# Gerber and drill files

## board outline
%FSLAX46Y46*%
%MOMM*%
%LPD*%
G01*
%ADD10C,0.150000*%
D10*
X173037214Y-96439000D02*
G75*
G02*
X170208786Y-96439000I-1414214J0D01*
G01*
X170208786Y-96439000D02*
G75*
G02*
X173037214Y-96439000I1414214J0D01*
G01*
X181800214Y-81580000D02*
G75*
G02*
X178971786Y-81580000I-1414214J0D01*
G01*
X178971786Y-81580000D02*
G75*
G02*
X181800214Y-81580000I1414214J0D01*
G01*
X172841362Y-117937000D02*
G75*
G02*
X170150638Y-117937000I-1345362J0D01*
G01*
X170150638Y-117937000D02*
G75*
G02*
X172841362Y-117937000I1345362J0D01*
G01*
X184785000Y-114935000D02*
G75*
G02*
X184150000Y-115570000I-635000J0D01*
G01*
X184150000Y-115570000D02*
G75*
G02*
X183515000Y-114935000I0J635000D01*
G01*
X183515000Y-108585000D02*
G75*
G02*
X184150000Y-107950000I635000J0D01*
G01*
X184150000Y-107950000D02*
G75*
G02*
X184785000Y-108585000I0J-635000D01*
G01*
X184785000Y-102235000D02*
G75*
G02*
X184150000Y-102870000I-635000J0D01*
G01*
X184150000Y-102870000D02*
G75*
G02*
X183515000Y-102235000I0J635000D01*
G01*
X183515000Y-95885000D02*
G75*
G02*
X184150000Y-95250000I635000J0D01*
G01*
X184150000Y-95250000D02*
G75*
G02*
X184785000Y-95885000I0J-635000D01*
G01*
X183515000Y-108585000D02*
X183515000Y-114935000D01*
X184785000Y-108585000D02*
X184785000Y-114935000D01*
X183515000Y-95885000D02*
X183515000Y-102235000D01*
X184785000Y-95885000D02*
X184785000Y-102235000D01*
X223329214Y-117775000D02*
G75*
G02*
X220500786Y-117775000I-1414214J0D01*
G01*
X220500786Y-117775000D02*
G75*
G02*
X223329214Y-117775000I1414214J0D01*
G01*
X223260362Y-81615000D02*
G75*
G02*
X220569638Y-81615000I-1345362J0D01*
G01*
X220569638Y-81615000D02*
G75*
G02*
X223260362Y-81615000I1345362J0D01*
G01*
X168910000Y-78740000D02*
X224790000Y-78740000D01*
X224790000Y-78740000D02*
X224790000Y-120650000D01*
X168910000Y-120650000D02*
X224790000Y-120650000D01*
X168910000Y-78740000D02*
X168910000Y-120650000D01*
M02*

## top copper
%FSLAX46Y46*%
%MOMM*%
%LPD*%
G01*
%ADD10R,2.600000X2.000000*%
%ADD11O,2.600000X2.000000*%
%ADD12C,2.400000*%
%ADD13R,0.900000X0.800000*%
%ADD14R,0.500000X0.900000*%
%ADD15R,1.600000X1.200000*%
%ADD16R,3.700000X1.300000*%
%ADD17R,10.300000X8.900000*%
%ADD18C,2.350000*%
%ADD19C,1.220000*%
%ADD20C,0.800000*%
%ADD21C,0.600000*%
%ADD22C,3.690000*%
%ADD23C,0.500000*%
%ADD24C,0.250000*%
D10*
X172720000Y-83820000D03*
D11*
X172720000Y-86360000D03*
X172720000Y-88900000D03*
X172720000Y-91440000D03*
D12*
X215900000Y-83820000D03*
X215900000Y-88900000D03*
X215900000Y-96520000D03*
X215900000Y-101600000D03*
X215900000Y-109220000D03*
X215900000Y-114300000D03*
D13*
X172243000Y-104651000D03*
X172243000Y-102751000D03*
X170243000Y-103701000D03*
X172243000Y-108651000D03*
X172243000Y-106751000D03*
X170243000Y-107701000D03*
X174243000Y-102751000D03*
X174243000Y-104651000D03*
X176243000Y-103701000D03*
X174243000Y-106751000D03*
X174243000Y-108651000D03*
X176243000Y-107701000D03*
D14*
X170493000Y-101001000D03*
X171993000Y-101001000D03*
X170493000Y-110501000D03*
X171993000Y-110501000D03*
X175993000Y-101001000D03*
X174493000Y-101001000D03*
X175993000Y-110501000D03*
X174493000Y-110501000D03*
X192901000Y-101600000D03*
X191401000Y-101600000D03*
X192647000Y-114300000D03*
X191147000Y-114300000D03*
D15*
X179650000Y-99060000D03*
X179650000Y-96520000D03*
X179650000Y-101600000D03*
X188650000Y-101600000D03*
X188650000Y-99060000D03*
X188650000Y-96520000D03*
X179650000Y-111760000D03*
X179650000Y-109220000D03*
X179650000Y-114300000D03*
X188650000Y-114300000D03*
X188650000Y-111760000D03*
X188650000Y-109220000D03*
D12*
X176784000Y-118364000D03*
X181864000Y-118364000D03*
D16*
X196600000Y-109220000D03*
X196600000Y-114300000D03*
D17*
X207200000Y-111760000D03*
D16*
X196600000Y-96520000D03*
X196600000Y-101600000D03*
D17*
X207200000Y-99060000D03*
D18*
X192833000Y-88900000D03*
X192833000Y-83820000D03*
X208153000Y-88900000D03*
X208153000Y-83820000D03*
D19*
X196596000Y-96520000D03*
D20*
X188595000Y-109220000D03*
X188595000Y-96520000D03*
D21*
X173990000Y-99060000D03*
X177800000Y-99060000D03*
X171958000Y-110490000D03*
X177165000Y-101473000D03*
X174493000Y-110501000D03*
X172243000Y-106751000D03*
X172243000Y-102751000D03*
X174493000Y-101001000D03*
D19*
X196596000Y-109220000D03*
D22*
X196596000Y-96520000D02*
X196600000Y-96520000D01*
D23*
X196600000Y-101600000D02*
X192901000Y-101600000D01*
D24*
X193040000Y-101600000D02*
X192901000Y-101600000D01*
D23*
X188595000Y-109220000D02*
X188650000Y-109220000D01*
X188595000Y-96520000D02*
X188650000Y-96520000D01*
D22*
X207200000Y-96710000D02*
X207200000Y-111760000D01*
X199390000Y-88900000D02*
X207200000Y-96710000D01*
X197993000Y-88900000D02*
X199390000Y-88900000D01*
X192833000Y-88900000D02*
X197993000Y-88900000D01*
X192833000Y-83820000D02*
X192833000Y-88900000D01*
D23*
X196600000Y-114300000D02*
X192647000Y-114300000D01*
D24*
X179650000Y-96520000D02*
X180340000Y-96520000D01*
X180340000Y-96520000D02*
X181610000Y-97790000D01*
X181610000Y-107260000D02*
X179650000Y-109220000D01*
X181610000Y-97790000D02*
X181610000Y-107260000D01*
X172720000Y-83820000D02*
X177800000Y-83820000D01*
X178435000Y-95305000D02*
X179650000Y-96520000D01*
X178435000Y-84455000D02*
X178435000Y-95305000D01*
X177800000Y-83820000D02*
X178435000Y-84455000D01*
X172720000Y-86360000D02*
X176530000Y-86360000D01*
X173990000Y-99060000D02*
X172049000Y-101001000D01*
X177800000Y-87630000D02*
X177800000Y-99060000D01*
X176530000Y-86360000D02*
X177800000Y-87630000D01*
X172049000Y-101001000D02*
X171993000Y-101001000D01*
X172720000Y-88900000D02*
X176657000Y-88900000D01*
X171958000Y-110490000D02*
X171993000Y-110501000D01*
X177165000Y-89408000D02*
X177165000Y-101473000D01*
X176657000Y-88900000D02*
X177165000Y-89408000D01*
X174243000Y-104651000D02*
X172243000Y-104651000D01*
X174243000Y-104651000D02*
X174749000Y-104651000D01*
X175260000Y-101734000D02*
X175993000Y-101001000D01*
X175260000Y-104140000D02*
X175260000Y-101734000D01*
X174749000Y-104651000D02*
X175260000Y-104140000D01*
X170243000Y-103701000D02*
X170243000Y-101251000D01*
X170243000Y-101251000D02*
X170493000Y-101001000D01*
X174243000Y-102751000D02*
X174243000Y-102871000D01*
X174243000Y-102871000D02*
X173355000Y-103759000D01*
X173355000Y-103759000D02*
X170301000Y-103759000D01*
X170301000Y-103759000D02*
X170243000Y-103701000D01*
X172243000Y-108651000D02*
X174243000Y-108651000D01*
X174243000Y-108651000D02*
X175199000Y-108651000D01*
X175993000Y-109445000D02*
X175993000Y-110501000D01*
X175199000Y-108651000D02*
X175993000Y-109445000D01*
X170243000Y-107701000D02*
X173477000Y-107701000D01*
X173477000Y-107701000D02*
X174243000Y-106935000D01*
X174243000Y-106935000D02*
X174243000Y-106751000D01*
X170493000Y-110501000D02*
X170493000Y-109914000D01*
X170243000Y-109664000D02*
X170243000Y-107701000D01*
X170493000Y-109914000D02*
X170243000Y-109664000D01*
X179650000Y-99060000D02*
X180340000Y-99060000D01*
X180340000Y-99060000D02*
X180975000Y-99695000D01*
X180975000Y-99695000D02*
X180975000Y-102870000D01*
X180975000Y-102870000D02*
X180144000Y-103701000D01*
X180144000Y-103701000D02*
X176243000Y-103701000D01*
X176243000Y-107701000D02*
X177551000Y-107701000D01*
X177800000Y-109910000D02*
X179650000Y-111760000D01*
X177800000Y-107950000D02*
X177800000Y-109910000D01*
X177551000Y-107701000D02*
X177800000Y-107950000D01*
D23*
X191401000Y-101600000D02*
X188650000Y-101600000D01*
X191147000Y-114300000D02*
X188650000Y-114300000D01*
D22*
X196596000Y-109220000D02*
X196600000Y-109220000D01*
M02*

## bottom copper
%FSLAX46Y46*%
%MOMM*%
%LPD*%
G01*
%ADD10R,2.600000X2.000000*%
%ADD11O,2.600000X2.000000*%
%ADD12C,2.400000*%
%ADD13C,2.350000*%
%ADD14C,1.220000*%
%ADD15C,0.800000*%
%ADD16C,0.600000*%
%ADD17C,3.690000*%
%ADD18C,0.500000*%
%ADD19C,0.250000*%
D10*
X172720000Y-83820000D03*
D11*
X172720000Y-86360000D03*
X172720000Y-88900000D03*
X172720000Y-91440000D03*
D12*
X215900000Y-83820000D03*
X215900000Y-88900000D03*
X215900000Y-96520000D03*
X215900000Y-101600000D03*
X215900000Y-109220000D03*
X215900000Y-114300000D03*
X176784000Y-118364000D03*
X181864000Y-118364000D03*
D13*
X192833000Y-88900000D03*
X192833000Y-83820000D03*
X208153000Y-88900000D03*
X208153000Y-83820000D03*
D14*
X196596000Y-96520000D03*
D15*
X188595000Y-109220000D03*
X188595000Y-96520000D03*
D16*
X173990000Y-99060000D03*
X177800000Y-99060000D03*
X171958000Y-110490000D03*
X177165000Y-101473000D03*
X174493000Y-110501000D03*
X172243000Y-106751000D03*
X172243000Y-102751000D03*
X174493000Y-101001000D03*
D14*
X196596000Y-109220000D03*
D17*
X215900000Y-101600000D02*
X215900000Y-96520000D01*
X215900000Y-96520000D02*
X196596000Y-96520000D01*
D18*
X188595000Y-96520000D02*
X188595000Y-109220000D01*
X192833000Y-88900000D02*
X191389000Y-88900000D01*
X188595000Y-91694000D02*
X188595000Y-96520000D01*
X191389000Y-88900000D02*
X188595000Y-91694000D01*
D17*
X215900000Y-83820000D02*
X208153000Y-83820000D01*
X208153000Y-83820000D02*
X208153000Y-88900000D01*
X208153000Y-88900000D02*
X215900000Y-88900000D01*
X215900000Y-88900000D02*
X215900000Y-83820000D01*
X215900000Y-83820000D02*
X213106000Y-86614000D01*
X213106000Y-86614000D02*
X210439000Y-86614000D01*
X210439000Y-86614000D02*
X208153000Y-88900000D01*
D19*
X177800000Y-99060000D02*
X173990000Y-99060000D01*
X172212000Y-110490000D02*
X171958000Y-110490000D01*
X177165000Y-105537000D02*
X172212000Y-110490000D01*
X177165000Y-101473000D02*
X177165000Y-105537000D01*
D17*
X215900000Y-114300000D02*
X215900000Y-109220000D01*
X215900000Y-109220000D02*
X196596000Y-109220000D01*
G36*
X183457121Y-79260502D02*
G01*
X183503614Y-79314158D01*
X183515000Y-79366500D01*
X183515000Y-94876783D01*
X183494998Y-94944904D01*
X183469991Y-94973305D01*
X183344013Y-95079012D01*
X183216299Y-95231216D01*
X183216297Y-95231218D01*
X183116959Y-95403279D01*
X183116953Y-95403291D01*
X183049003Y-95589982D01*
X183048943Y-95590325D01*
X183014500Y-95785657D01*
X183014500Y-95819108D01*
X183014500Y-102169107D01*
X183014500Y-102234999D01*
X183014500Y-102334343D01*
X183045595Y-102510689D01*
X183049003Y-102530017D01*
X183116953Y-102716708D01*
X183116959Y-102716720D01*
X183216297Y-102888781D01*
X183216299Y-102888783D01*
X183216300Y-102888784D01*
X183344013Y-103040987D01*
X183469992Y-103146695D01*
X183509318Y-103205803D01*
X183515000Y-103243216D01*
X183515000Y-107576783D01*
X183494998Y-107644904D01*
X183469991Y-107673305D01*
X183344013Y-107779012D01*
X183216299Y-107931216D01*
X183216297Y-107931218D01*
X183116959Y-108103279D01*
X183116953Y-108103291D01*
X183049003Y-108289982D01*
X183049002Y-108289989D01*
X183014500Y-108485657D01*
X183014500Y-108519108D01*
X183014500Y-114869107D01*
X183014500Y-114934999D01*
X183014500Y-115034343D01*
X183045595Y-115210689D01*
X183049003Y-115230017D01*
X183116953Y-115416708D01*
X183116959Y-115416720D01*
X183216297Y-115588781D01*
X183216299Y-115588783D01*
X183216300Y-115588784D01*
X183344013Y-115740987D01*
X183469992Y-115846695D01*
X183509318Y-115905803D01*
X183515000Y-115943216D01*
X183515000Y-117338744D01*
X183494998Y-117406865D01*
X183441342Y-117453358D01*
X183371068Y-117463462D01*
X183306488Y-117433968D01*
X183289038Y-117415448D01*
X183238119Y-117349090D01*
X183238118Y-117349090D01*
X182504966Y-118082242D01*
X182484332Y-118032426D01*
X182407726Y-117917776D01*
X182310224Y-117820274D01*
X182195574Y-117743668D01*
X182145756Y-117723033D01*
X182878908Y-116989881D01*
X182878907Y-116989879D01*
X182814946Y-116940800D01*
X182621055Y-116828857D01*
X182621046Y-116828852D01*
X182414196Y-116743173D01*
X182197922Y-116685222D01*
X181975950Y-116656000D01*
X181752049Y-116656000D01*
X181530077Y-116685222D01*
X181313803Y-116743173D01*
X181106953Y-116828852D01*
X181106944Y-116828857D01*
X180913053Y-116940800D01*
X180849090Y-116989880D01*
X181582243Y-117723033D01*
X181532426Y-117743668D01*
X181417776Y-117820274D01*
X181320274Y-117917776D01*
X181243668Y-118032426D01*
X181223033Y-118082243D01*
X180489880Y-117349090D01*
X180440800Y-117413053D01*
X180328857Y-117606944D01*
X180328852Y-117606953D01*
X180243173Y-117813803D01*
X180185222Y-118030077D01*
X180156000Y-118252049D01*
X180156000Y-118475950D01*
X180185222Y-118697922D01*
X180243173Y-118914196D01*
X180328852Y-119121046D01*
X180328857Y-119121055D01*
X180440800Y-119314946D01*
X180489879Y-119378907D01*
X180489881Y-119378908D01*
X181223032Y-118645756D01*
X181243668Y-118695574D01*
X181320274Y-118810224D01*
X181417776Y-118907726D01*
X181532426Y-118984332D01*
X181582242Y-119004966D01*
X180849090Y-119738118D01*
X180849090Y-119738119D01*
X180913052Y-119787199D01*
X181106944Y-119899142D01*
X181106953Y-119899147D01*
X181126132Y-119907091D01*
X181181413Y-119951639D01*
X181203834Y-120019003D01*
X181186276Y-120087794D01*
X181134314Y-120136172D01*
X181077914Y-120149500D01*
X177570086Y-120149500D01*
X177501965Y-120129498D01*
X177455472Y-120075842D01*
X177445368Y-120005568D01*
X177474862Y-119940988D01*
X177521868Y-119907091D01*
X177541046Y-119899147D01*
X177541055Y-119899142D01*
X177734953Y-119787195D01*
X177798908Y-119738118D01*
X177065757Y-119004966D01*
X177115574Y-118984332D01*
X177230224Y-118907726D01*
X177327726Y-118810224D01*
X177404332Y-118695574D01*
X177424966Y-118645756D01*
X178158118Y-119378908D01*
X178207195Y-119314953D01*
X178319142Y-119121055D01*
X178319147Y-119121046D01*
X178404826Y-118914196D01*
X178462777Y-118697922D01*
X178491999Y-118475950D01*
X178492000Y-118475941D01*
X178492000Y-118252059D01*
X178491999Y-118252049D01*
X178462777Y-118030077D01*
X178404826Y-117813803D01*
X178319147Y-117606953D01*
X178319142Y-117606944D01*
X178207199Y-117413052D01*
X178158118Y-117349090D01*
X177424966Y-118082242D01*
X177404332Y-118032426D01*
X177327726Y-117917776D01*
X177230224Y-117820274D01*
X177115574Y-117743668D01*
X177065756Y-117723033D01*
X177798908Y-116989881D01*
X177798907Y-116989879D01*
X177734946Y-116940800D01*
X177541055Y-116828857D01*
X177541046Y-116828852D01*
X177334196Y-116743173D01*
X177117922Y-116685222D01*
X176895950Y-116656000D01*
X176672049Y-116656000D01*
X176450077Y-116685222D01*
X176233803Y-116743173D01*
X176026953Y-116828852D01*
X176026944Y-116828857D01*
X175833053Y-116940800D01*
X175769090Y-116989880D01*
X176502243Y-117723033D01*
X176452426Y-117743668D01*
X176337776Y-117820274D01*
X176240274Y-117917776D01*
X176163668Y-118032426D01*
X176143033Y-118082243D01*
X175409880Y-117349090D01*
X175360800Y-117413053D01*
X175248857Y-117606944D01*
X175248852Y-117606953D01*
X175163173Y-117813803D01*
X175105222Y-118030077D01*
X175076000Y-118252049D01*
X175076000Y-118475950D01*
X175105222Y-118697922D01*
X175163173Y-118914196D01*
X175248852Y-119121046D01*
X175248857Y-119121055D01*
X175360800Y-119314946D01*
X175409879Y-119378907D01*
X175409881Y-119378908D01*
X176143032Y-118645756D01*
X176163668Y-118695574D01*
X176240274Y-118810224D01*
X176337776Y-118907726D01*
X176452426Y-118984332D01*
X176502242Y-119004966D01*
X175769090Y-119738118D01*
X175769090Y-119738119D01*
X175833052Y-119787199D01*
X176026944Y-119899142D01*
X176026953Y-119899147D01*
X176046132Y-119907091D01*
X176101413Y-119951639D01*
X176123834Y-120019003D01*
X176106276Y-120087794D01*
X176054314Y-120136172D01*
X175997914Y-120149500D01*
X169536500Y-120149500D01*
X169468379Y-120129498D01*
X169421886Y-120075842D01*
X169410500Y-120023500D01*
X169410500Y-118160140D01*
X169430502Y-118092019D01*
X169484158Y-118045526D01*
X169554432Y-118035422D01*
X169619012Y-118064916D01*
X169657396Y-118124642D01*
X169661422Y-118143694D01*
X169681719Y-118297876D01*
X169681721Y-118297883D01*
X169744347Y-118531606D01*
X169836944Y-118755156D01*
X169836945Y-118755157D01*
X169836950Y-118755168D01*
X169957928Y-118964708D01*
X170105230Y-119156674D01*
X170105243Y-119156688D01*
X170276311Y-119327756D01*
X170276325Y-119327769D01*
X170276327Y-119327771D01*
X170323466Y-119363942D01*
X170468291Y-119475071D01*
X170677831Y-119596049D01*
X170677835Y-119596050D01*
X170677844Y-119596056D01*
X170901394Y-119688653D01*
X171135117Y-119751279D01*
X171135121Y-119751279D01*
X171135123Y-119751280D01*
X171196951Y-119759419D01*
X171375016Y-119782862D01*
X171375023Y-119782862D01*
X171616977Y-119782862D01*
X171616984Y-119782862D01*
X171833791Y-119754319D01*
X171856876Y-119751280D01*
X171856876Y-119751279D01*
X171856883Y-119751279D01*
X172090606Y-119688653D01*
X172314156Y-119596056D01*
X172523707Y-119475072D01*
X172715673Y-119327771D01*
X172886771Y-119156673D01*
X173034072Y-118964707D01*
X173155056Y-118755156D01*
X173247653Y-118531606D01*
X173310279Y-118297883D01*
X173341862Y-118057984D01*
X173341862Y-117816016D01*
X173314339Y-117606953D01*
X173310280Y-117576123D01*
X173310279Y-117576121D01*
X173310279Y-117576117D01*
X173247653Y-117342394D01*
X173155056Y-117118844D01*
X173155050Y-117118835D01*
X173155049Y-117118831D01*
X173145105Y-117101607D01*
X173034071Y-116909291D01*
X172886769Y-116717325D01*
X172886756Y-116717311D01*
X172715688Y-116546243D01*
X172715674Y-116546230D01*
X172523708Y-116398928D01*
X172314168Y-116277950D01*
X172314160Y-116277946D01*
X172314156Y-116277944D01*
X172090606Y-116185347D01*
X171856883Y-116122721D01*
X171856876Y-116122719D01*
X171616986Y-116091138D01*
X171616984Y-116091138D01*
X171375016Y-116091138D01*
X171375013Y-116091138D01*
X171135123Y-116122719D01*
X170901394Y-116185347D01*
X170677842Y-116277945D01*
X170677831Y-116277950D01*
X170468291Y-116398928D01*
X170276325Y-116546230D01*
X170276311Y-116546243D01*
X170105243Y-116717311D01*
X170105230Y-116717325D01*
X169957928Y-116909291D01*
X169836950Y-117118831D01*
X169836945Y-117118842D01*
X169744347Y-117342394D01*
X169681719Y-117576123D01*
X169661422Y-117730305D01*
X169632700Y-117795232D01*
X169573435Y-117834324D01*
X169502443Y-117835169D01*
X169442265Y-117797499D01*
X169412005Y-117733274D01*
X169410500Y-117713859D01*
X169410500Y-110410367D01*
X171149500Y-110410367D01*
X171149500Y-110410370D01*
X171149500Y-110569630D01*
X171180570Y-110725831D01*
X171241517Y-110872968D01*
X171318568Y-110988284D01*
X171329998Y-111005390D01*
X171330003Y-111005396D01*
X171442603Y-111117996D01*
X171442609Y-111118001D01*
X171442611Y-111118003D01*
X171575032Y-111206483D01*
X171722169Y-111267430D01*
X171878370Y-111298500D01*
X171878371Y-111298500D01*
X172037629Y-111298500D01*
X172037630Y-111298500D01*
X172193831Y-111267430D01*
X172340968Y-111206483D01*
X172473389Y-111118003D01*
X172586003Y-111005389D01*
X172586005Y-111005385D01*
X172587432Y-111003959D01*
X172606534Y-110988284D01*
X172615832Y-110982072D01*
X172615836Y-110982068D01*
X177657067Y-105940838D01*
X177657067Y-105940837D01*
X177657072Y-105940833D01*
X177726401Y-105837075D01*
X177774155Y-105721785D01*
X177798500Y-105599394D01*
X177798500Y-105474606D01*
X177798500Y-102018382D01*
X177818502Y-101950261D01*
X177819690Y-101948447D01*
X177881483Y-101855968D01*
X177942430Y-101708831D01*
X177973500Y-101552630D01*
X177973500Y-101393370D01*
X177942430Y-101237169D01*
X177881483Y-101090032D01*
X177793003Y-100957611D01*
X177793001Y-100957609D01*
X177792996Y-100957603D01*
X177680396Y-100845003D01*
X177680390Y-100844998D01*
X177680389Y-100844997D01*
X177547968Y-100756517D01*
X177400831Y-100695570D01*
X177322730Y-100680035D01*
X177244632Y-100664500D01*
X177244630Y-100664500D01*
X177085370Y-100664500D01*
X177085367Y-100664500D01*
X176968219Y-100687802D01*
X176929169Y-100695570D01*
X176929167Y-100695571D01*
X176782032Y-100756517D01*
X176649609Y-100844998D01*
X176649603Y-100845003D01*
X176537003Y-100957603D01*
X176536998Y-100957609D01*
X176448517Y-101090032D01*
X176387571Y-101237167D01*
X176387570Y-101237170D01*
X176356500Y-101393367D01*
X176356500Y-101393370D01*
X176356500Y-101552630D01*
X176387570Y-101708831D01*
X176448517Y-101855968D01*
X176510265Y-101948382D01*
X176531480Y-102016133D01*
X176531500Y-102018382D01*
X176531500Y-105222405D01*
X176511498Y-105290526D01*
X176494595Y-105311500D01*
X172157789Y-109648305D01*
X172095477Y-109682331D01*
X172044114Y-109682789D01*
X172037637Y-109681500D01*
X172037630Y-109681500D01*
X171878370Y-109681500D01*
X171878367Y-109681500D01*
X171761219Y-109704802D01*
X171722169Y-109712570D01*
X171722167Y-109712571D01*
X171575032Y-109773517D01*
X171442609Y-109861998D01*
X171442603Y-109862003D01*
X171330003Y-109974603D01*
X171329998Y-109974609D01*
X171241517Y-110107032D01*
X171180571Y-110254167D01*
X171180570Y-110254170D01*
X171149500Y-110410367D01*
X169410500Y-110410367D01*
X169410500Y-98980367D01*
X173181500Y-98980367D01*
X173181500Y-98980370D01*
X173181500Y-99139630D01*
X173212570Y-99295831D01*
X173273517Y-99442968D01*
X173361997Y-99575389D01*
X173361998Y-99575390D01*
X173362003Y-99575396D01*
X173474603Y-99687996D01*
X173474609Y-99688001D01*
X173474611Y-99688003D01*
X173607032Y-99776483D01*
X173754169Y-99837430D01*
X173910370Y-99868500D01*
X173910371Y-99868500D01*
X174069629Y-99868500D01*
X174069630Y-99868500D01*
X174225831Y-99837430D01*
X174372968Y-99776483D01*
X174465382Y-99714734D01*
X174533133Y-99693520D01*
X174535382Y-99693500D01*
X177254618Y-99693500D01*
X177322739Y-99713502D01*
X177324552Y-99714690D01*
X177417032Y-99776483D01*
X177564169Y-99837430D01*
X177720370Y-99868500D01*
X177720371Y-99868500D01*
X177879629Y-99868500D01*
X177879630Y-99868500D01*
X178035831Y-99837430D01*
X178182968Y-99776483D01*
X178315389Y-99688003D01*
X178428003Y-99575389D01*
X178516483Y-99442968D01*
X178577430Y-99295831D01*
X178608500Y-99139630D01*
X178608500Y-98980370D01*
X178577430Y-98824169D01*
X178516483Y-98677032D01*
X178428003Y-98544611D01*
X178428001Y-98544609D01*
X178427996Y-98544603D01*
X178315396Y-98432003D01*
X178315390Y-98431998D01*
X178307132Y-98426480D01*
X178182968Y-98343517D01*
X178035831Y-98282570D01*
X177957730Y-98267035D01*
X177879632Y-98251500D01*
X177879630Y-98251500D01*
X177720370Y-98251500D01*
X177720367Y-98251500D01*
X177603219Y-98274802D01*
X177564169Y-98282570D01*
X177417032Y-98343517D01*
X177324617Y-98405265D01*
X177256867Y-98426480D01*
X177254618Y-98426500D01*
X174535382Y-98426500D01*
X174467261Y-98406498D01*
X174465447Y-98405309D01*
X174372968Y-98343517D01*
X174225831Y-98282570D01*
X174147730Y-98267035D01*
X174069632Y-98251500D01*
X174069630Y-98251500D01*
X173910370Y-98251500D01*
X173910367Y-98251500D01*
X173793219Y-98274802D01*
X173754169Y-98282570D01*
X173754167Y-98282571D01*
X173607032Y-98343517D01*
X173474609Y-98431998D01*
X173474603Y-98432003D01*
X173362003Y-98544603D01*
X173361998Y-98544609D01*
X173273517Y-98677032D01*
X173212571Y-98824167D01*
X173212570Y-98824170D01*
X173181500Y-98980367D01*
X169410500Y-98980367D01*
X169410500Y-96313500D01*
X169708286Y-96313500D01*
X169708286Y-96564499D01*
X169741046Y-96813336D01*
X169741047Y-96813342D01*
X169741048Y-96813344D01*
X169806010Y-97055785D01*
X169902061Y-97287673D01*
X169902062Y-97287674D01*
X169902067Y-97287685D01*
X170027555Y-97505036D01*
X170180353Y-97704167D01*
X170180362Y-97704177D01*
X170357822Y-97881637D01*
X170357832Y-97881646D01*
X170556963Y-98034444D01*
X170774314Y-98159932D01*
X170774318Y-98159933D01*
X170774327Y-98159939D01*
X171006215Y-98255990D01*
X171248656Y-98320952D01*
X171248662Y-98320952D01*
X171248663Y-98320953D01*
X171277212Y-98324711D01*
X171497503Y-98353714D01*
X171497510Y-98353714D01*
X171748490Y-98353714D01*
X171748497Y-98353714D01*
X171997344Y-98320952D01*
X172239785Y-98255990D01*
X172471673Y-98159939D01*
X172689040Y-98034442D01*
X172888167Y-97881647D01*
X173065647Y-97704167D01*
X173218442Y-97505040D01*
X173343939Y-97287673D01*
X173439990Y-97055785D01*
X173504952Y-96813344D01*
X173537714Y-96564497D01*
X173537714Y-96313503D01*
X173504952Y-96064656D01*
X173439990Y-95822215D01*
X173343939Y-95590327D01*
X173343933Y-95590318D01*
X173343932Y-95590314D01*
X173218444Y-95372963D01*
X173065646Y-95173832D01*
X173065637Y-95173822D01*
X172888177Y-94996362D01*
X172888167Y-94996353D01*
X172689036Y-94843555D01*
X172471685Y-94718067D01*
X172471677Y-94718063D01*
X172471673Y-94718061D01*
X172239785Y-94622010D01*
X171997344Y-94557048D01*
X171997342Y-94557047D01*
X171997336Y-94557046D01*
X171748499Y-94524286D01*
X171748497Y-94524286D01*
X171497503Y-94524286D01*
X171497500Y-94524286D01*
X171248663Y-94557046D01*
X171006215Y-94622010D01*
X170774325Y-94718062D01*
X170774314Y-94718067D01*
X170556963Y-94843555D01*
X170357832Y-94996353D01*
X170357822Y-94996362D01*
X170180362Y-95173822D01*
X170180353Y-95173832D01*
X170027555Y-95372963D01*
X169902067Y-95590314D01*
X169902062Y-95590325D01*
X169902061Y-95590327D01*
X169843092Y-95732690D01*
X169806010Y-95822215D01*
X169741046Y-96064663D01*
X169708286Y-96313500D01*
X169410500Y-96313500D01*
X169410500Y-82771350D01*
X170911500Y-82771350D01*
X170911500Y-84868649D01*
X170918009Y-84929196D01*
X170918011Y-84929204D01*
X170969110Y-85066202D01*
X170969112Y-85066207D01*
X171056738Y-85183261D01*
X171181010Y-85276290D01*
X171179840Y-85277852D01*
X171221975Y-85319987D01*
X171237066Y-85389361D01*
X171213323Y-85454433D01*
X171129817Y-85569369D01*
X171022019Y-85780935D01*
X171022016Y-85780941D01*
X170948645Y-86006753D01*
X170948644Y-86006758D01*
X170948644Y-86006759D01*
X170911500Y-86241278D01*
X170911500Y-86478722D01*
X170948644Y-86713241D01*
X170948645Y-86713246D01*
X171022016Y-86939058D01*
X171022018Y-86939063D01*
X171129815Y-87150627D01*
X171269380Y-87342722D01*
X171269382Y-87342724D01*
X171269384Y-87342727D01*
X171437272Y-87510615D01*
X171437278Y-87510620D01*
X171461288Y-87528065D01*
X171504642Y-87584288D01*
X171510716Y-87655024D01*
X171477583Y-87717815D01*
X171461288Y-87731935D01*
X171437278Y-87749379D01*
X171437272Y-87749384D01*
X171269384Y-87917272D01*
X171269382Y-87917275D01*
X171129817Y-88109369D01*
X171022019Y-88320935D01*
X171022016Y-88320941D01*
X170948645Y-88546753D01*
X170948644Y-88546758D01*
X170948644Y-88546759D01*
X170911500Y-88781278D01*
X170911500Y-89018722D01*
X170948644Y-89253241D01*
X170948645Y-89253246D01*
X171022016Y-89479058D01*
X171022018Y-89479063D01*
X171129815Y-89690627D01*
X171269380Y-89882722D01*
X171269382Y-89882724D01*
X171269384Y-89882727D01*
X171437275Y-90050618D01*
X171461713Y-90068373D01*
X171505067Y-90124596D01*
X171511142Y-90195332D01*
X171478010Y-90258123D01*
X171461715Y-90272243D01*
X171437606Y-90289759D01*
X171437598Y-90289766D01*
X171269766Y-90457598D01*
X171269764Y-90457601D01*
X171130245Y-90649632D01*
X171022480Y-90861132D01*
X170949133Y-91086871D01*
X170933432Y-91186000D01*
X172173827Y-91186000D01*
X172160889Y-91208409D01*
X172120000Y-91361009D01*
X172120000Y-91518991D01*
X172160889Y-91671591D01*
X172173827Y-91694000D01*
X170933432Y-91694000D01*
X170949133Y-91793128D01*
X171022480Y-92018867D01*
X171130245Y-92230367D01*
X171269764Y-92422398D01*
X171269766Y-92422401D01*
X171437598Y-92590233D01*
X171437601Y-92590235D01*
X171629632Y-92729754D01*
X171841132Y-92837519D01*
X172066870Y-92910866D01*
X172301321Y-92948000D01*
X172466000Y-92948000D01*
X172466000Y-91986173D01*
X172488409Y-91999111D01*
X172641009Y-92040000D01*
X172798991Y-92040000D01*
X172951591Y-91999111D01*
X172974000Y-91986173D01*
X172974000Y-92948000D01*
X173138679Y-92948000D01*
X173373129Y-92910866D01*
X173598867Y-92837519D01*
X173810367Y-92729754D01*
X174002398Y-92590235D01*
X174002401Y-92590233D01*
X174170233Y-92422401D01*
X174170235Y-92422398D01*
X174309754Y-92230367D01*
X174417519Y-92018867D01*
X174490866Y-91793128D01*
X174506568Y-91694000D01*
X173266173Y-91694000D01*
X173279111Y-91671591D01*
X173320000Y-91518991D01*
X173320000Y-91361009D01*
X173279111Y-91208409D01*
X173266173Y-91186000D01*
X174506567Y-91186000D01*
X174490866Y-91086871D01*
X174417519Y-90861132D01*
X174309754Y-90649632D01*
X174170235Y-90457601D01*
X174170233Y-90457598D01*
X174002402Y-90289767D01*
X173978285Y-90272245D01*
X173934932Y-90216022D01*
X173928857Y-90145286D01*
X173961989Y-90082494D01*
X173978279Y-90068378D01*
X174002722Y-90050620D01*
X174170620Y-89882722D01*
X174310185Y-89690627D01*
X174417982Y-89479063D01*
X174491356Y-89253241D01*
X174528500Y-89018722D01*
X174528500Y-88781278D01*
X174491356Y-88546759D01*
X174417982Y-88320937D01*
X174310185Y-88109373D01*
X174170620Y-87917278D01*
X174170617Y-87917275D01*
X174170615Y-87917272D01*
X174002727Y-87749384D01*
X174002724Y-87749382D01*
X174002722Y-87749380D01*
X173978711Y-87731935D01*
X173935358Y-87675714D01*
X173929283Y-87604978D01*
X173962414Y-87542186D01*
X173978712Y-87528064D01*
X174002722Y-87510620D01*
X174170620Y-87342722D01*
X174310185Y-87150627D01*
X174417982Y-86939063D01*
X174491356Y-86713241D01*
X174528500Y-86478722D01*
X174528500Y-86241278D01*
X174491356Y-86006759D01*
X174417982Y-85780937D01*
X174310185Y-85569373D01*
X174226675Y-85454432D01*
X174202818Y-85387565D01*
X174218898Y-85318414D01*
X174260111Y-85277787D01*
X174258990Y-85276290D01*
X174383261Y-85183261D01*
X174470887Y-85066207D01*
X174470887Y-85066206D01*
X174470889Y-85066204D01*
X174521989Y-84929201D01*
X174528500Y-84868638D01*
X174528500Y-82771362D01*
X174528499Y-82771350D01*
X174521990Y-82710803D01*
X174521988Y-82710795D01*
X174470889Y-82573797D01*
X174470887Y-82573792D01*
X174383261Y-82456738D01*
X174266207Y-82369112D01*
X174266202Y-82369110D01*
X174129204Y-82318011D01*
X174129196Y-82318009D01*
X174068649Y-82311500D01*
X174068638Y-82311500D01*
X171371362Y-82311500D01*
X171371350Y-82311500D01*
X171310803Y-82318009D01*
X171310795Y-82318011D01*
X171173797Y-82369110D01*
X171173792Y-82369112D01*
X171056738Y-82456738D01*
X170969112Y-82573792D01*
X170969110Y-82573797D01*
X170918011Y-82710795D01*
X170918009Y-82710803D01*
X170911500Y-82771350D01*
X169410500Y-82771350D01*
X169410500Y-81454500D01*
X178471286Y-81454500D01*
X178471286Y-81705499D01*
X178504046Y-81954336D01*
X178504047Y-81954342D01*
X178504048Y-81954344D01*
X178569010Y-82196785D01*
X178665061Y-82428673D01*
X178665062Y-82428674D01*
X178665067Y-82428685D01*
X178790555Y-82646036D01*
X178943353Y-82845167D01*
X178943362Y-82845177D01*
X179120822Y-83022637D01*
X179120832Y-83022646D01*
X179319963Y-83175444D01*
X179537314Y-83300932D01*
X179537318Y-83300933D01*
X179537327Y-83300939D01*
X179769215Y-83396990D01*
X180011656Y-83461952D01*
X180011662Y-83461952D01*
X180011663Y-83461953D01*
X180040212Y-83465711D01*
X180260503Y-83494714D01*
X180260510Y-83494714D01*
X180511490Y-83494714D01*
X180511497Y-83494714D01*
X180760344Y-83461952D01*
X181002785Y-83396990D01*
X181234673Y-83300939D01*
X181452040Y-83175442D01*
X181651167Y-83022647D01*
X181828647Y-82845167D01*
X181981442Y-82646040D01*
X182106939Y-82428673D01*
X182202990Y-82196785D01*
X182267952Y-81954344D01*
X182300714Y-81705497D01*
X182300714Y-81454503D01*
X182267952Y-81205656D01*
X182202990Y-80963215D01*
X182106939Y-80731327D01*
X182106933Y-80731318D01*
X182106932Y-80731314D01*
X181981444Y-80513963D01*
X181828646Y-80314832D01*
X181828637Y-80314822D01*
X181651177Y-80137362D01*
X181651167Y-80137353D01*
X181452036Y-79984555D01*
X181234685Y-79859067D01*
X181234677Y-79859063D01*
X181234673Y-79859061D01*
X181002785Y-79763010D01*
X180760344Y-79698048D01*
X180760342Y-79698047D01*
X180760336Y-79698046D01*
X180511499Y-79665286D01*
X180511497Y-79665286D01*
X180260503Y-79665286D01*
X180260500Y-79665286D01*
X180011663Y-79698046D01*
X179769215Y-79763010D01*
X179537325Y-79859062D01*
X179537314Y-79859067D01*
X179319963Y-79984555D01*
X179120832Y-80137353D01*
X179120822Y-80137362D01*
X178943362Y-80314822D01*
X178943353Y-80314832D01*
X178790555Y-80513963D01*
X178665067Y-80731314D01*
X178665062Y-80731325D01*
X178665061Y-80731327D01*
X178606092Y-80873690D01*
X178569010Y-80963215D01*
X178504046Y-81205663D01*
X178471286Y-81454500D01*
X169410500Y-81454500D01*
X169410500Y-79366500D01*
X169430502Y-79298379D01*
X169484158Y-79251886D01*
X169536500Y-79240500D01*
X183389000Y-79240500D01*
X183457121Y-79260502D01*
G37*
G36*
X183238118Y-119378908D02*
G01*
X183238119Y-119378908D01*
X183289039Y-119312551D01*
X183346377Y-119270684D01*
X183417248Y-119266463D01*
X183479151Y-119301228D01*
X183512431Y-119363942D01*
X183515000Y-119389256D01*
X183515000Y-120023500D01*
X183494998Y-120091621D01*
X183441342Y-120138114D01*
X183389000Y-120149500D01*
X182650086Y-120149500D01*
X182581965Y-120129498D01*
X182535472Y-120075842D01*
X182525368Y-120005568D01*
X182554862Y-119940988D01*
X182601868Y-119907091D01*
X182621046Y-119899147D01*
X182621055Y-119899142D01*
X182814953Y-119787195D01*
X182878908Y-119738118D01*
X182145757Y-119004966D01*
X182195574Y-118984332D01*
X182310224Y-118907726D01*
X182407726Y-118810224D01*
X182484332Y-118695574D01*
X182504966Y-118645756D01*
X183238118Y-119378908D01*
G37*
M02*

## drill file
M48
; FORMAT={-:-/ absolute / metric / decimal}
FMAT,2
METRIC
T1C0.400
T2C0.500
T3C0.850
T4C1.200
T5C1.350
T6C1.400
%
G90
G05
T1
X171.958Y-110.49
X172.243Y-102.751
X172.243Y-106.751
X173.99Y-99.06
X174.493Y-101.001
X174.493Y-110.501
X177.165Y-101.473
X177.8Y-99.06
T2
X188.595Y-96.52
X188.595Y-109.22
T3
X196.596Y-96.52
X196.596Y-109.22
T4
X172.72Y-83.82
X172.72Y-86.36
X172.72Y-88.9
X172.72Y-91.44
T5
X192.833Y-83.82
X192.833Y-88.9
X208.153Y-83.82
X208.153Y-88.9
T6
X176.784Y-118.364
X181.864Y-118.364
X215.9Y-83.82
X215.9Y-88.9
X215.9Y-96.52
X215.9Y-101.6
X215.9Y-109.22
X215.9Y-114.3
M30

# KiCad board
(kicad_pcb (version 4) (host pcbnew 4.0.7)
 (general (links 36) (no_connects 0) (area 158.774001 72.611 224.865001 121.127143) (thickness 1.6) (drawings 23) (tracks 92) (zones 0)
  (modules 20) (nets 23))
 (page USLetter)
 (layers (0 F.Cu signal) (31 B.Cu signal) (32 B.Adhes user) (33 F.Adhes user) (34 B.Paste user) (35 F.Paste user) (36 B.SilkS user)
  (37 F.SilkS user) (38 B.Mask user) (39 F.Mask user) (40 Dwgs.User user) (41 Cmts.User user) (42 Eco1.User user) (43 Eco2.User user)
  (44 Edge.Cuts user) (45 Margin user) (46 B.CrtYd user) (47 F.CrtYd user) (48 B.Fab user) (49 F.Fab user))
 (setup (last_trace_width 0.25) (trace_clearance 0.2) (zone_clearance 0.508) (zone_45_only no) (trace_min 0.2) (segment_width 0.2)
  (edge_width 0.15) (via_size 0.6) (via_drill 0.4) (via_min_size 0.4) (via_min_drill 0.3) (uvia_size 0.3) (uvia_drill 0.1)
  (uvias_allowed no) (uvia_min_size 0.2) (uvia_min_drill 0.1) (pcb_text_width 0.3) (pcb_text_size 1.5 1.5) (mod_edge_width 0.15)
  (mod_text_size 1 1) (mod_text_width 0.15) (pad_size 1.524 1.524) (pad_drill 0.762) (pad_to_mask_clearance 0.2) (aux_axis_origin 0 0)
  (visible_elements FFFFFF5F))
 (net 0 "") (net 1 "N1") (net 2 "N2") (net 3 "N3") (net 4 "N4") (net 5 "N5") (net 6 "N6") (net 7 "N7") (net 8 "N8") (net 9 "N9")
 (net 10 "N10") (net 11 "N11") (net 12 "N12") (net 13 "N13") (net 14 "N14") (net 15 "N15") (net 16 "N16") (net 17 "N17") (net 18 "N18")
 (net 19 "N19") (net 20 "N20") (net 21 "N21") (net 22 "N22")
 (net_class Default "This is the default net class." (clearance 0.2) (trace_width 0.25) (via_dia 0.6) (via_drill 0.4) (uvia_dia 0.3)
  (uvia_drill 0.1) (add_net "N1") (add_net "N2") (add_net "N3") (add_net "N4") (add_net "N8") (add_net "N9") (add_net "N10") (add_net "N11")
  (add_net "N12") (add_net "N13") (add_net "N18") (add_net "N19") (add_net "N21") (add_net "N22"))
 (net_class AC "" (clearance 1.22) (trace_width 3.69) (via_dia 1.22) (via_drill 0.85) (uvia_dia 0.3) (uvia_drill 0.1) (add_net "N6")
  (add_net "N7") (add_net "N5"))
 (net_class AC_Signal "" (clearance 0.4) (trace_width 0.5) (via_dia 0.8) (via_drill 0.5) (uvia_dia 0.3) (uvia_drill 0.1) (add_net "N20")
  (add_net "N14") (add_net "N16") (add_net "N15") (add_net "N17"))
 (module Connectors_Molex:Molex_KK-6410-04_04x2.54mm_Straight (layer F.Cu) (at 172.72 83.82 270)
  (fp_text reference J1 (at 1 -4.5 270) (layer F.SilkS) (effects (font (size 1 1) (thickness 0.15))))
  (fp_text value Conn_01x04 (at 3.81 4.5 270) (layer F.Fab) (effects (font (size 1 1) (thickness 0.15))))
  (pad 1 thru_hole rect (at 0 0 270) (size 2 2.6) (drill 1.2) (layers *.Cu *.Mask) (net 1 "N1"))
  (pad 2 thru_hole oval (at 2.54 0 270) (size 2 2.6) (drill 1.2) (layers *.Cu *.Mask) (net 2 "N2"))
  (pad 3 thru_hole oval (at 5.08 0 270) (size 2 2.6) (drill 1.2) (layers *.Cu *.Mask) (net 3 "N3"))
  (pad 4 thru_hole oval (at 7.62 0 270) (size 2 2.6) (drill 1.2) (layers *.Cu *.Mask) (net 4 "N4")))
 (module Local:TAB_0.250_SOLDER (layer F.Cu) (at 215.9 88.9 90)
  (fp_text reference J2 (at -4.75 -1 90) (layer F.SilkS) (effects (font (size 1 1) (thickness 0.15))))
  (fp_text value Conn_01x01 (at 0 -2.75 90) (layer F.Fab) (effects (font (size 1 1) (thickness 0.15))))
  (pad 1 thru_hole circle (at 5.08 0 90) (size 2.4 2.4) (drill 1.4) (layers *.Cu *.Mask) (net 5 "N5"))
  (pad 1 thru_hole circle (at 0 0 90) (size 2.4 2.4) (drill 1.4) (layers *.Cu *.Mask) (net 5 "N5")))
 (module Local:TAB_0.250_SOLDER (layer F.Cu) (at 215.9 101.6 90)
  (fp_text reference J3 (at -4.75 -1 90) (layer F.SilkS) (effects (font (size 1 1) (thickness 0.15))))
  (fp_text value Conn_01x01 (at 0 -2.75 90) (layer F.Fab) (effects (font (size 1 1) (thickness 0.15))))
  (pad 1 thru_hole circle (at 5.08 0 90) (size 2.4 2.4) (drill 1.4) (layers *.Cu *.Mask) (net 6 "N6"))
  (pad 1 thru_hole circle (at 0 0 90) (size 2.4 2.4) (drill 1.4) (layers *.Cu *.Mask) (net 6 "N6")))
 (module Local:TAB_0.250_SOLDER (layer F.Cu) (at 215.9 114.3 90)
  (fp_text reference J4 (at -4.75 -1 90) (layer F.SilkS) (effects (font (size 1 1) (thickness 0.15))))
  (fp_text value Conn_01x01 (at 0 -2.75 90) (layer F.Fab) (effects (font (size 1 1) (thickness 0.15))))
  (pad 1 thru_hole circle (at 5.08 0 90) (size 2.4 2.4) (drill 1.4) (layers *.Cu *.Mask) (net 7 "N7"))
  (pad 1 thru_hole circle (at 0 0 90) (size 2.4 2.4) (drill 1.4) (layers *.Cu *.Mask) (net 7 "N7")))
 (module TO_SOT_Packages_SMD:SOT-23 (layer F.Cu) (at 171.243 103.701 180)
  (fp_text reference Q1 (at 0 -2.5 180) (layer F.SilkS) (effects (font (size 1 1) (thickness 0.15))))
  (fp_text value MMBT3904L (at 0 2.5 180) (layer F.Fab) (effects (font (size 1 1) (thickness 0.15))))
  (pad 1 smd rect (at -1 -0.95 180) (size 0.9 0.8) (layers F.Cu F.Paste F.Mask) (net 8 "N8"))
  (pad 2 smd rect (at -1 0.95 180) (size 0.9 0.8) (layers F.Cu F.Paste F.Mask) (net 4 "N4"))
  (pad 3 smd rect (at 1 0 180) (size 0.9 0.8) (layers F.Cu F.Paste F.Mask) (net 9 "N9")))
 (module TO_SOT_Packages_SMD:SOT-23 (layer F.Cu) (at 171.243 107.701 180)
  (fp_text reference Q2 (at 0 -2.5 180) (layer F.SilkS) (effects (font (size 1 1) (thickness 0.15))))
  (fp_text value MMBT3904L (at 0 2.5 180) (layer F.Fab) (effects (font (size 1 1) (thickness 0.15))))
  (pad 1 smd rect (at -1 -0.95 180) (size 0.9 0.8) (layers F.Cu F.Paste F.Mask) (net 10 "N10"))
  (pad 2 smd rect (at -1 0.95 180) (size 0.9 0.8) (layers F.Cu F.Paste F.Mask) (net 4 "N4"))
  (pad 3 smd rect (at 1 0 180) (size 0.9 0.8) (layers F.Cu F.Paste F.Mask) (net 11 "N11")))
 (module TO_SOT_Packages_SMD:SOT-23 (layer F.Cu) (at 175.243 103.701)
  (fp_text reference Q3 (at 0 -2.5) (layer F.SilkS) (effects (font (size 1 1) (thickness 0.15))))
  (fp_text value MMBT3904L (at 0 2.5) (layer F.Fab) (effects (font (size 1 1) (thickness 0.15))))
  (pad 1 smd rect (at -1 -0.95) (size 0.9 0.8) (layers F.Cu F.Paste F.Mask) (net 9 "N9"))
  (pad 2 smd rect (at -1 0.95) (size 0.9 0.8) (layers F.Cu F.Paste F.Mask) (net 8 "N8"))
  (pad 3 smd rect (at 1 0) (size 0.9 0.8) (layers F.Cu F.Paste F.Mask) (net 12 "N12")))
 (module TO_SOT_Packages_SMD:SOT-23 (layer F.Cu) (at 175.243 107.701)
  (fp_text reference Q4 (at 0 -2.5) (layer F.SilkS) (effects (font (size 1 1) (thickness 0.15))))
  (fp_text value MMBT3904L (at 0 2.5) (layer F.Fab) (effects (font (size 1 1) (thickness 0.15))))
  (pad 1 smd rect (at -1 -0.95) (size 0.9 0.8) (layers F.Cu F.Paste F.Mask) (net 11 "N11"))
  (pad 2 smd rect (at -1 0.95) (size 0.9 0.8) (layers F.Cu F.Paste F.Mask) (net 10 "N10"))
  (pad 3 smd rect (at 1 0) (size 0.9 0.8) (layers F.Cu F.Paste F.Mask) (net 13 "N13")))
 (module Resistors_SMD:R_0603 (layer F.Cu) (at 171.243 101.001)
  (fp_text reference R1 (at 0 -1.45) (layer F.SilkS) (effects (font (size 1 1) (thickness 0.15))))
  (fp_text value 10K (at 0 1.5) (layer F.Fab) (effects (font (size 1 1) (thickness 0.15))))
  (pad 1 smd rect (at -0.75 0) (size 0.5 0.9) (layers F.Cu F.Paste F.Mask) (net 9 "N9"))
  (pad 2 smd rect (at 0.75 0) (size 0.5 0.9) (layers F.Cu F.Paste F.Mask) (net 2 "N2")))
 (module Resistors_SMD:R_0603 (layer F.Cu) (at 171.243 110.501)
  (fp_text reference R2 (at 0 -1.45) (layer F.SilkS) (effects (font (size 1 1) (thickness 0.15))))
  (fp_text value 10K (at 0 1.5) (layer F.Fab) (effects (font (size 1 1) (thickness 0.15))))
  (pad 1 smd rect (at -0.75 0) (size 0.5 0.9) (layers F.Cu F.Paste F.Mask) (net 11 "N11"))
  (pad 2 smd rect (at 0.75 0) (size 0.5 0.9) (layers F.Cu F.Paste F.Mask) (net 3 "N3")))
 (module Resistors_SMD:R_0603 (layer F.Cu) (at 175.243 101.001 180)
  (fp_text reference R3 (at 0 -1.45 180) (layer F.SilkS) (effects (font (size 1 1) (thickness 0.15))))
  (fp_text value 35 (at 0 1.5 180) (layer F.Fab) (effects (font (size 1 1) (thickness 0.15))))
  (pad 1 smd rect (at -0.75 0 180) (size 0.5 0.9) (layers F.Cu F.Paste F.Mask) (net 8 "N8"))
  (pad 2 smd rect (at 0.75 0 180) (size 0.5 0.9) (layers F.Cu F.Paste F.Mask) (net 4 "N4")))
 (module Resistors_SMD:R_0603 (layer F.Cu) (at 175.243 110.501 180)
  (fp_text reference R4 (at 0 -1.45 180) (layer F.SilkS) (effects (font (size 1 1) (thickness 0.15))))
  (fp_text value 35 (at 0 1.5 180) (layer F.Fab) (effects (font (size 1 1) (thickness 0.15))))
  (pad 1 smd rect (at -0.75 0 180) (size 0.5 0.9) (layers F.Cu F.Paste F.Mask) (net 10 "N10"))
  (pad 2 smd rect (at 0.75 0 180) (size 0.5 0.9) (layers F.Cu F.Paste F.Mask) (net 4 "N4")))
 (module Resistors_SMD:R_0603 (layer F.Cu) (at 192.151 101.6 180)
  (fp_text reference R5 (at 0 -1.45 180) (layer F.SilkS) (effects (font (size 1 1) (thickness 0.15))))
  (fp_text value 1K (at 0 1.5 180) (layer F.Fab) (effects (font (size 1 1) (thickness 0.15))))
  (pad 1 smd rect (at -0.75 0 180) (size 0.5 0.9) (layers F.Cu F.Paste F.Mask) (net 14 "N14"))
  (pad 2 smd rect (at 0.75 0 180) (size 0.5 0.9) (layers F.Cu F.Paste F.Mask) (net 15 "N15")))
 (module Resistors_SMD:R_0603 (layer F.Cu) (at 191.897 114.3 180)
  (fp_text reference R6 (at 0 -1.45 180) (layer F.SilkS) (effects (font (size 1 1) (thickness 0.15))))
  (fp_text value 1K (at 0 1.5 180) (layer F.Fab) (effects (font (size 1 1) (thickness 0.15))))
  (pad 1 smd rect (at -0.75 0 180) (size 0.5 0.9) (layers F.Cu F.Paste F.Mask) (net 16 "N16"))
  (pad 2 smd rect (at 0.75 0 180) (size 0.5 0.9) (layers F.Cu F.Paste F.Mask) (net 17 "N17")))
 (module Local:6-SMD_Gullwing (layer F.Cu) (at 184.15 99.06 270)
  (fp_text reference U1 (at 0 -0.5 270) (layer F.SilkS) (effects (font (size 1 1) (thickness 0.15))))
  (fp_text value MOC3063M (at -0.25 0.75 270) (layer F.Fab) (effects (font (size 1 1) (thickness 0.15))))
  (pad 2 smd rect (at 0 4.5 270) (size 1.2 1.6) (layers F.Cu F.Paste F.Mask) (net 12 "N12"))
  (pad 1 smd rect (at -2.54 4.5 270) (size 1.2 1.6) (layers F.Cu F.Paste F.Mask) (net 1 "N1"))
  (pad 3 smd rect (at 2.54 4.5 270) (size 1.2 1.6) (layers F.Cu F.Paste F.Mask) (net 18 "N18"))
  (pad 4 smd rect (at 2.54 -4.5 270) (size 1.2 1.6) (layers F.Cu F.Paste F.Mask) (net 15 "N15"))
  (pad 5 smd rect (at 0 -4.5 270) (size 1.2 1.6) (layers F.Cu F.Paste F.Mask) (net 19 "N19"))
  (pad 6 smd rect (at -2.54 -4.5 270) (size 1.2 1.6) (layers F.Cu F.Paste F.Mask) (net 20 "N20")))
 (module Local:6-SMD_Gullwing (layer F.Cu) (at 184.15 111.76 270)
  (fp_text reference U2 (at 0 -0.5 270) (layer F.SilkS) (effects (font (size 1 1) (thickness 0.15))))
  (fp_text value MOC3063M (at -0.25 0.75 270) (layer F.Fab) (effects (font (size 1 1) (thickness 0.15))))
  (pad 2 smd rect (at 0 4.5 270) (size 1.2 1.6) (layers F.Cu F.Paste F.Mask) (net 13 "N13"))
  (pad 1 smd rect (at -2.54 4.5 270) (size 1.2 1.6) (layers F.Cu F.Paste F.Mask) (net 1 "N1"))
  (pad 3 smd rect (at 2.54 4.5 270) (size 1.2 1.6) (layers F.Cu F.Paste F.Mask) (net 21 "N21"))
  (pad 4 smd rect (at 2.54 -4.5 270) (size 1.2 1.6) (layers F.Cu F.Paste F.Mask) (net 17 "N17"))
  (pad 5 smd rect (at 0 -4.5 270) (size 1.2 1.6) (layers F.Cu F.Paste F.Mask) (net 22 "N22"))
  (pad 6 smd rect (at -2.54 -4.5 270) (size 1.2 1.6) (layers F.Cu F.Paste F.Mask) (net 20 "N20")))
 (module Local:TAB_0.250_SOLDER (layer F.Cu) (at 181.864 118.364 180)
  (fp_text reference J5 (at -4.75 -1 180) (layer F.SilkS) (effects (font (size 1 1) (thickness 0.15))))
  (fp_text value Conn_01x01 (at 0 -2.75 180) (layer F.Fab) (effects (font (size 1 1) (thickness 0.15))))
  (pad 1 thru_hole circle (at 5.08 0 180) (size 2.4 2.4) (drill 1.4) (layers *.Cu *.Mask) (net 4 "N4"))
  (pad 1 thru_hole circle (at 0 0 180) (size 2.4 2.4) (drill 1.4) (layers *.Cu *.Mask) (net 4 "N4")))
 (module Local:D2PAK (layer F.Cu) (at 203.2 111.76 180)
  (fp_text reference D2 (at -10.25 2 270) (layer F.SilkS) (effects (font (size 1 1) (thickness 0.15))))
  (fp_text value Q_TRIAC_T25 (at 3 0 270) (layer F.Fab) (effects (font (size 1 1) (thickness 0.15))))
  (pad 1 smd rect (at 6.6 2.54 180) (size 3.7 1.3) (layers F.Cu F.Paste F.Mask) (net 7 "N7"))
  (pad 3 smd rect (at 6.6 -2.54 180) (size 3.7 1.3) (layers F.Cu F.Paste F.Mask) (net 16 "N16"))
  (pad 2 smd rect (at -4 0 180) (size 10.3 8.9) (layers F.Cu F.Paste F.Mask) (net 20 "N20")))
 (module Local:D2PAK (layer F.Cu) (at 203.2 99.06 180)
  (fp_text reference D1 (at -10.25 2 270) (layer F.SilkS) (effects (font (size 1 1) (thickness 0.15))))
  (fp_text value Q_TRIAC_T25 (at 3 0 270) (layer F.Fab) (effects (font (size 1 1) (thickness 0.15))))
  (pad 1 smd rect (at 6.6 2.54 180) (size 3.7 1.3) (layers F.Cu F.Paste F.Mask) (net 6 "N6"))
  (pad 3 smd rect (at 6.6 -2.54 180) (size 3.7 1.3) (layers F.Cu F.Paste F.Mask) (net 14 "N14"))
  (pad 2 smd rect (at -4 0 180) (size 10.3 8.9) (layers F.Cu F.Paste F.Mask) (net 20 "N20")))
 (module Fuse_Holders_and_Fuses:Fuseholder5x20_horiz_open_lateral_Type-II (layer F.Cu) (at 208.153 88.9 180)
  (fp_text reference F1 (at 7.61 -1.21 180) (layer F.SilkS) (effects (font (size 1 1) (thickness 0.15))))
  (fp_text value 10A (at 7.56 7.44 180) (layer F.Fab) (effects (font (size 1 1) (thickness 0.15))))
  (pad 2 thru_hole circle (at 15.32 0 180) (size 2.35 2.35) (drill 1.35) (layers *.Cu *.Mask) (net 20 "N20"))
  (pad 2 thru_hole circle (at 15.32 5.08 180) (size 2.35 2.35) (drill 1.35) (layers *.Cu *.Mask) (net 20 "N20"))
  (pad 1 thru_hole circle (at 0 0 180) (size 2.35 2.35) (drill 1.35) (layers *.Cu *.Mask) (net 5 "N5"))
  (pad 1 thru_hole circle (at 0 5.08 180) (size 2.35 2.35) (drill 1.35) (layers *.Cu *.Mask) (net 5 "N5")))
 (gr_circle (center 171.623 96.439) (end 172.623 97.439) (layer Edge.Cuts) (width 0.15))
 (gr_circle (center 180.386 81.58) (end 181.386 82.58) (layer Edge.Cuts) (width 0.15))
 (gr_circle (center 171.496 117.937) (end 172.496 118.837) (layer Edge.Cuts) (width 0.15))
 (gr_arc (start 184.15 114.935) (end 184.785 114.935) (angle 90) (layer Edge.Cuts) (width 0.15))
 (gr_arc (start 184.15 114.935) (end 184.15 115.57) (angle 90) (layer Edge.Cuts) (width 0.15))
 (gr_arc (start 184.15 108.585) (end 183.515 108.585) (angle 90) (layer Edge.Cuts) (width 0.15))
 (gr_arc (start 184.15 108.585) (end 184.15 107.95) (angle 90) (layer Edge.Cuts) (width 0.15))
 (gr_arc (start 184.15 102.235) (end 184.785 102.235) (angle 90) (layer Edge.Cuts) (width 0.15))
 (gr_arc (start 184.15 102.235) (end 184.15 102.87) (angle 90) (layer Edge.Cuts) (width 0.15))
 (gr_arc (start 184.15 95.885) (end 183.515 95.885) (angle 90) (layer Edge.Cuts) (width 0.15))
 (gr_arc (start 184.15 95.885) (end 184.15 95.25) (angle 90) (layer Edge.Cuts) (width 0.15))
 (gr_line (start 183.515 108.585) (end 183.515 114.935) (angle 90) (layer Edge.Cuts) (width 0.15))
 (gr_line (start 184.785 108.585) (end 184.785 114.935) (angle 90) (layer Edge.Cuts) (width 0.15))
 (gr_line (start 183.515 95.885) (end 183.515 102.235) (angle 90) (layer Edge.Cuts) (width 0.15))
 (gr_line (start 184.785 95.885) (end 184.785 102.235) (angle 90) (layer Edge.Cuts) (width 0.15))
 (gr_circle (center 221.915 117.775) (end 222.915 118.775) (layer Edge.Cuts) (width 0.15))
 (gr_circle (center 221.915 81.615) (end 222.915 82.515) (layer Edge.Cuts) (width 0.15))
 (gr_line (start 168.91 78.74) (end 224.79 78.74) (angle 90) (layer Edge.Cuts) (width 0.15))
 (gr_line (start 224.79 78.74) (end 224.79 120.65) (angle 90) (layer Edge.Cuts) (width 0.15))
 (gr_line (start 168.91 120.65) (end 224.79 120.65) (angle 90) (layer Edge.Cuts) (width 0.15))
 (gr_line (start 168.91 78.74) (end 168.91 120.65) (angle 90) (layer Edge.Cuts) (width 0.15))
 (segment (start 215.9 101.6) (end 215.9 96.52) (width 3.69) (layer B.Cu) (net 6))
 (segment (start 215.9 96.52) (end 196.596 96.52) (width 3.69) (layer B.Cu) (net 6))
 (via (at 196.596 96.52) (size 1.22) (drill 0.85) (layers F.Cu B.Cu) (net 6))
 (segment (start 196.596 96.52) (end 196.6 96.52) (width 3.69) (layer F.Cu) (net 6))
 (segment (start 196.6 101.6) (end 192.901 101.6) (width 0.5) (layer F.Cu) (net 14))
 (segment (start 193.04 101.6) (end 192.901 101.6) (width 0.25) (layer F.Cu) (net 14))
 (segment (start 188.595 96.52) (end 188.595 109.22) (width 0.5) (layer B.Cu) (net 20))
 (segment (start 188.595 109.22) (end 188.65 109.22) (width 0.5) (layer F.Cu) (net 20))
 (via (at 188.595 109.22) (size 0.8) (drill 0.5) (layers F.Cu B.Cu) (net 20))
 (segment (start 192.833 88.9) (end 191.389 88.9) (width 0.5) (layer B.Cu) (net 20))
 (segment (start 188.595 96.52) (end 188.65 96.52) (width 0.5) (layer F.Cu) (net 20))
 (via (at 188.595 96.52) (size 0.8) (drill 0.5) (layers F.Cu B.Cu) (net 20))
 (segment (start 188.595 91.694) (end 188.595 96.52) (width 0.5) (layer B.Cu) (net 20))
 (segment (start 191.389 88.9) (end 188.595 91.694) (width 0.5) (layer B.Cu) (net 20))
 (segment (start 207.2 96.71) (end 207.2 111.76) (width 3.69) (layer F.Cu) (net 20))
 (segment (start 199.39 88.9) (end 207.2 96.71) (width 3.69) (layer F.Cu) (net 20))
 (segment (start 197.993 88.9) (end 199.39 88.9) (width 3.69) (layer F.Cu) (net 20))
 (segment (start 192.833 88.9) (end 197.993 88.9) (width 3.69) (layer F.Cu) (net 20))
 (segment (start 192.833 83.82) (end 192.833 88.9) (width 3.69) (layer F.Cu) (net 20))
 (segment (start 196.6 114.3) (end 192.647 114.3) (width 0.5) (layer F.Cu) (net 16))
 (segment (start 215.9 83.82) (end 208.153 83.82) (width 3.69) (layer B.Cu) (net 5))
 (segment (start 208.153 83.82) (end 208.153 88.9) (width 3.69) (layer B.Cu) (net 5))
 (segment (start 208.153 88.9) (end 215.9 88.9) (width 3.69) (layer B.Cu) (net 5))
 (segment (start 215.9 88.9) (end 215.9 83.82) (width 3.69) (layer B.Cu) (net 5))
 (segment (start 215.9 83.82) (end 213.106 86.614) (width 3.69) (layer B.Cu) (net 5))
 (segment (start 213.106 86.614) (end 210.439 86.614) (width 3.69) (layer B.Cu) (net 5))
 (segment (start 210.439 86.614) (end 208.153 88.9) (width 3.69) (layer B.Cu) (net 5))
 (segment (start 179.65 96.52) (end 180.34 96.52) (width 0.25) (layer F.Cu) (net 1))
 (segment (start 180.34 96.52) (end 181.61 97.79) (width 0.25) (layer F.Cu) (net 1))
 (segment (start 181.61 107.26) (end 179.65 109.22) (width 0.25) (layer F.Cu) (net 1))
 (segment (start 181.61 97.79) (end 181.61 107.26) (width 0.25) (layer F.Cu) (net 1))
 (segment (start 172.72 83.82) (end 177.8 83.82) (width 0.25) (layer F.Cu) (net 1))
 (segment (start 178.435 95.305) (end 179.65 96.52) (width 0.25) (layer F.Cu) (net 1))
 (segment (start 178.435 84.455) (end 178.435 95.305) (width 0.25) (layer F.Cu) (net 1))
 (segment (start 177.8 83.82) (end 178.435 84.455) (width 0.25) (layer F.Cu) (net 1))
 (segment (start 172.72 86.36) (end 176.53 86.36) (width 0.25) (layer F.Cu) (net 2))
 (segment (start 173.99 99.06) (end 172.049 101.001) (width 0.25) (layer F.Cu) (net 2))
 (via (at 173.99 99.06) (size 0.6) (drill 0.4) (layers F.Cu B.Cu) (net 2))
 (segment (start 177.8 99.06) (end 173.99 99.06) (width 0.25) (layer B.Cu) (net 2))
 (via (at 177.8 99.06) (size 0.6) (drill 0.4) (layers F.Cu B.Cu) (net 2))
 (segment (start 177.8 87.63) (end 177.8 99.06) (width 0.25) (layer F.Cu) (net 2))
 (segment (start 176.53 86.36) (end 177.8 87.63) (width 0.25) (layer F.Cu) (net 2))
 (segment (start 172.049 101.001) (end 171.993 101.001) (width 0.25) (layer F.Cu) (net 2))
 (segment (start 172.72 88.9) (end 176.657 88.9) (width 0.25) (layer F.Cu) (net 3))
 (segment (start 171.958 110.49) (end 171.993 110.501) (width 0.25) (layer F.Cu) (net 3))
 (via (at 171.958 110.49) (size 0.6) (drill 0.4) (layers F.Cu B.Cu) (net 3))
 (segment (start 172.212 110.49) (end 171.958 110.49) (width 0.25) (layer B.Cu) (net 3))
 (segment (start 177.165 105.537) (end 172.212 110.49) (width 0.25) (layer B.Cu) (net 3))
 (segment (start 177.165 101.473) (end 177.165 105.537) (width 0.25) (layer B.Cu) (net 3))
 (via (at 177.165 101.473) (size 0.6) (drill 0.4) (layers F.Cu B.Cu) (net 3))
 (segment (start 177.165 89.408) (end 177.165 101.473) (width 0.25) (layer F.Cu) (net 3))
 (segment (start 176.657 88.9) (end 177.165 89.408) (width 0.25) (layer F.Cu) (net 3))
 (via (at 174.493 110.501) (size 0.6) (drill 0.4) (layers F.Cu B.Cu) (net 4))
 (via (at 172.243 106.751) (size 0.6) (drill 0.4) (layers F.Cu B.Cu) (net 4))
 (via (at 172.243 102.751) (size 0.6) (drill 0.4) (layers F.Cu B.Cu) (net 4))
 (via (at 174.493 101.001) (size 0.6) (drill 0.4) (layers F.Cu B.Cu) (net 4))
 (segment (start 174.243 104.651) (end 172.243 104.651) (width 0.25) (layer F.Cu) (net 8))
 (segment (start 174.243 104.651) (end 174.749 104.651) (width 0.25) (layer F.Cu) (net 8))
 (segment (start 175.26 101.734) (end 175.993 101.001) (width 0.25) (layer F.Cu) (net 8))
 (segment (start 175.26 104.14) (end 175.26 101.734) (width 0.25) (layer F.Cu) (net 8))
 (segment (start 174.749 104.651) (end 175.26 104.14) (width 0.25) (layer F.Cu) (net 8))
 (segment (start 170.243 103.701) (end 170.243 101.251) (width 0.25) (layer F.Cu) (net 9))
 (segment (start 170.243 101.251) (end 170.493 101.001) (width 0.25) (layer F.Cu) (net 9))
 (segment (start 174.243 102.751) (end 174.243 102.871) (width 0.25) (layer F.Cu) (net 9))
 (segment (start 174.243 102.871) (end 173.355 103.759) (width 0.25) (layer F.Cu) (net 9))
 (segment (start 173.355 103.759) (end 170.301 103.759) (width 0.25) (layer F.Cu) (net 9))
 (segment (start 170.301 103.759) (end 170.243 103.701) (width 0.25) (layer F.Cu) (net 9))
 (segment (start 172.243 108.651) (end 174.243 108.651) (width 0.25) (layer F.Cu) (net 10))
 (segment (start 174.243 108.651) (end 175.199 108.651) (width 0.25) (layer F.Cu) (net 10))
 (segment (start 175.993 109.445) (end 175.993 110.501) (width 0.25) (layer F.Cu) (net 10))
 (segment (start 175.199 108.651) (end 175.993 109.445) (width 0.25) (layer F.Cu) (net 10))
 (segment (start 170.243 107.701) (end 173.477 107.701) (width 0.25) (layer F.Cu) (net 11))
 (segment (start 173.477 107.701) (end 174.243 106.935) (width 0.25) (layer F.Cu) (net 11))
 (segment (start 174.243 106.935) (end 174.243 106.751) (width 0.25) (layer F.Cu) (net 11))
 (segment (start 170.493 110.501) (end 170.493 109.914) (width 0.25) (layer F.Cu) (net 11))
 (segment (start 170.243 109.664) (end 170.243 107.701) (width 0.25) (layer F.Cu) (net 11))
 (segment (start 170.493 109.914) (end 170.243 109.664) (width 0.25) (layer F.Cu) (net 11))
 (segment (start 179.65 99.06) (end 180.34 99.06) (width 0.25) (layer F.Cu) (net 12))
 (segment (start 180.34 99.06) (end 180.975 99.695) (width 0.25) (layer F.Cu) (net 12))
 (segment (start 180.975 99.695) (end 180.975 102.87) (width 0.25) (layer F.Cu) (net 12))
 (segment (start 180.975 102.87) (end 180.144 103.701) (width 0.25) (layer F.Cu) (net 12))
 (segment (start 180.144 103.701) (end 176.243 103.701) (width 0.25) (layer F.Cu) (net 12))
 (segment (start 176.243 107.701) (end 177.551 107.701) (width 0.25) (layer F.Cu) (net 13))
 (segment (start 177.8 109.91) (end 179.65 111.76) (width 0.25) (layer F.Cu) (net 13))
 (segment (start 177.8 107.95) (end 177.8 109.91) (width 0.25) (layer F.Cu) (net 13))
 (segment (start 177.551 107.701) (end 177.8 107.95) (width 0.25) (layer F.Cu) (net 13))
 (segment (start 191.401 101.6) (end 188.65 101.6) (width 0.5) (layer F.Cu) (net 15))
 (segment (start 191.147 114.3) (end 188.65 114.3) (width 0.5) (layer F.Cu) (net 17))
 (segment (start 215.9 114.3) (end 215.9 109.22) (width 3.69) (layer B.Cu) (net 7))
 (segment (start 215.9 109.22) (end 196.596 109.22) (width 3.69) (layer B.Cu) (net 7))
 (via (at 196.596 109.22) (size 1.22) (drill 0.85) (layers F.Cu B.Cu) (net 7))
 (segment (start 196.596 109.22) (end 196.6 109.22) (width 3.69) (layer F.Cu) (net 7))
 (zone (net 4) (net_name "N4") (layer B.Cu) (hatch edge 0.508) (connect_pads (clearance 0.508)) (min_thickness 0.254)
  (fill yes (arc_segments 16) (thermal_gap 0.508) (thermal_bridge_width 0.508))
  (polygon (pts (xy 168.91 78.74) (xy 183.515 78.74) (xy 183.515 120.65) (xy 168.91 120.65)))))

